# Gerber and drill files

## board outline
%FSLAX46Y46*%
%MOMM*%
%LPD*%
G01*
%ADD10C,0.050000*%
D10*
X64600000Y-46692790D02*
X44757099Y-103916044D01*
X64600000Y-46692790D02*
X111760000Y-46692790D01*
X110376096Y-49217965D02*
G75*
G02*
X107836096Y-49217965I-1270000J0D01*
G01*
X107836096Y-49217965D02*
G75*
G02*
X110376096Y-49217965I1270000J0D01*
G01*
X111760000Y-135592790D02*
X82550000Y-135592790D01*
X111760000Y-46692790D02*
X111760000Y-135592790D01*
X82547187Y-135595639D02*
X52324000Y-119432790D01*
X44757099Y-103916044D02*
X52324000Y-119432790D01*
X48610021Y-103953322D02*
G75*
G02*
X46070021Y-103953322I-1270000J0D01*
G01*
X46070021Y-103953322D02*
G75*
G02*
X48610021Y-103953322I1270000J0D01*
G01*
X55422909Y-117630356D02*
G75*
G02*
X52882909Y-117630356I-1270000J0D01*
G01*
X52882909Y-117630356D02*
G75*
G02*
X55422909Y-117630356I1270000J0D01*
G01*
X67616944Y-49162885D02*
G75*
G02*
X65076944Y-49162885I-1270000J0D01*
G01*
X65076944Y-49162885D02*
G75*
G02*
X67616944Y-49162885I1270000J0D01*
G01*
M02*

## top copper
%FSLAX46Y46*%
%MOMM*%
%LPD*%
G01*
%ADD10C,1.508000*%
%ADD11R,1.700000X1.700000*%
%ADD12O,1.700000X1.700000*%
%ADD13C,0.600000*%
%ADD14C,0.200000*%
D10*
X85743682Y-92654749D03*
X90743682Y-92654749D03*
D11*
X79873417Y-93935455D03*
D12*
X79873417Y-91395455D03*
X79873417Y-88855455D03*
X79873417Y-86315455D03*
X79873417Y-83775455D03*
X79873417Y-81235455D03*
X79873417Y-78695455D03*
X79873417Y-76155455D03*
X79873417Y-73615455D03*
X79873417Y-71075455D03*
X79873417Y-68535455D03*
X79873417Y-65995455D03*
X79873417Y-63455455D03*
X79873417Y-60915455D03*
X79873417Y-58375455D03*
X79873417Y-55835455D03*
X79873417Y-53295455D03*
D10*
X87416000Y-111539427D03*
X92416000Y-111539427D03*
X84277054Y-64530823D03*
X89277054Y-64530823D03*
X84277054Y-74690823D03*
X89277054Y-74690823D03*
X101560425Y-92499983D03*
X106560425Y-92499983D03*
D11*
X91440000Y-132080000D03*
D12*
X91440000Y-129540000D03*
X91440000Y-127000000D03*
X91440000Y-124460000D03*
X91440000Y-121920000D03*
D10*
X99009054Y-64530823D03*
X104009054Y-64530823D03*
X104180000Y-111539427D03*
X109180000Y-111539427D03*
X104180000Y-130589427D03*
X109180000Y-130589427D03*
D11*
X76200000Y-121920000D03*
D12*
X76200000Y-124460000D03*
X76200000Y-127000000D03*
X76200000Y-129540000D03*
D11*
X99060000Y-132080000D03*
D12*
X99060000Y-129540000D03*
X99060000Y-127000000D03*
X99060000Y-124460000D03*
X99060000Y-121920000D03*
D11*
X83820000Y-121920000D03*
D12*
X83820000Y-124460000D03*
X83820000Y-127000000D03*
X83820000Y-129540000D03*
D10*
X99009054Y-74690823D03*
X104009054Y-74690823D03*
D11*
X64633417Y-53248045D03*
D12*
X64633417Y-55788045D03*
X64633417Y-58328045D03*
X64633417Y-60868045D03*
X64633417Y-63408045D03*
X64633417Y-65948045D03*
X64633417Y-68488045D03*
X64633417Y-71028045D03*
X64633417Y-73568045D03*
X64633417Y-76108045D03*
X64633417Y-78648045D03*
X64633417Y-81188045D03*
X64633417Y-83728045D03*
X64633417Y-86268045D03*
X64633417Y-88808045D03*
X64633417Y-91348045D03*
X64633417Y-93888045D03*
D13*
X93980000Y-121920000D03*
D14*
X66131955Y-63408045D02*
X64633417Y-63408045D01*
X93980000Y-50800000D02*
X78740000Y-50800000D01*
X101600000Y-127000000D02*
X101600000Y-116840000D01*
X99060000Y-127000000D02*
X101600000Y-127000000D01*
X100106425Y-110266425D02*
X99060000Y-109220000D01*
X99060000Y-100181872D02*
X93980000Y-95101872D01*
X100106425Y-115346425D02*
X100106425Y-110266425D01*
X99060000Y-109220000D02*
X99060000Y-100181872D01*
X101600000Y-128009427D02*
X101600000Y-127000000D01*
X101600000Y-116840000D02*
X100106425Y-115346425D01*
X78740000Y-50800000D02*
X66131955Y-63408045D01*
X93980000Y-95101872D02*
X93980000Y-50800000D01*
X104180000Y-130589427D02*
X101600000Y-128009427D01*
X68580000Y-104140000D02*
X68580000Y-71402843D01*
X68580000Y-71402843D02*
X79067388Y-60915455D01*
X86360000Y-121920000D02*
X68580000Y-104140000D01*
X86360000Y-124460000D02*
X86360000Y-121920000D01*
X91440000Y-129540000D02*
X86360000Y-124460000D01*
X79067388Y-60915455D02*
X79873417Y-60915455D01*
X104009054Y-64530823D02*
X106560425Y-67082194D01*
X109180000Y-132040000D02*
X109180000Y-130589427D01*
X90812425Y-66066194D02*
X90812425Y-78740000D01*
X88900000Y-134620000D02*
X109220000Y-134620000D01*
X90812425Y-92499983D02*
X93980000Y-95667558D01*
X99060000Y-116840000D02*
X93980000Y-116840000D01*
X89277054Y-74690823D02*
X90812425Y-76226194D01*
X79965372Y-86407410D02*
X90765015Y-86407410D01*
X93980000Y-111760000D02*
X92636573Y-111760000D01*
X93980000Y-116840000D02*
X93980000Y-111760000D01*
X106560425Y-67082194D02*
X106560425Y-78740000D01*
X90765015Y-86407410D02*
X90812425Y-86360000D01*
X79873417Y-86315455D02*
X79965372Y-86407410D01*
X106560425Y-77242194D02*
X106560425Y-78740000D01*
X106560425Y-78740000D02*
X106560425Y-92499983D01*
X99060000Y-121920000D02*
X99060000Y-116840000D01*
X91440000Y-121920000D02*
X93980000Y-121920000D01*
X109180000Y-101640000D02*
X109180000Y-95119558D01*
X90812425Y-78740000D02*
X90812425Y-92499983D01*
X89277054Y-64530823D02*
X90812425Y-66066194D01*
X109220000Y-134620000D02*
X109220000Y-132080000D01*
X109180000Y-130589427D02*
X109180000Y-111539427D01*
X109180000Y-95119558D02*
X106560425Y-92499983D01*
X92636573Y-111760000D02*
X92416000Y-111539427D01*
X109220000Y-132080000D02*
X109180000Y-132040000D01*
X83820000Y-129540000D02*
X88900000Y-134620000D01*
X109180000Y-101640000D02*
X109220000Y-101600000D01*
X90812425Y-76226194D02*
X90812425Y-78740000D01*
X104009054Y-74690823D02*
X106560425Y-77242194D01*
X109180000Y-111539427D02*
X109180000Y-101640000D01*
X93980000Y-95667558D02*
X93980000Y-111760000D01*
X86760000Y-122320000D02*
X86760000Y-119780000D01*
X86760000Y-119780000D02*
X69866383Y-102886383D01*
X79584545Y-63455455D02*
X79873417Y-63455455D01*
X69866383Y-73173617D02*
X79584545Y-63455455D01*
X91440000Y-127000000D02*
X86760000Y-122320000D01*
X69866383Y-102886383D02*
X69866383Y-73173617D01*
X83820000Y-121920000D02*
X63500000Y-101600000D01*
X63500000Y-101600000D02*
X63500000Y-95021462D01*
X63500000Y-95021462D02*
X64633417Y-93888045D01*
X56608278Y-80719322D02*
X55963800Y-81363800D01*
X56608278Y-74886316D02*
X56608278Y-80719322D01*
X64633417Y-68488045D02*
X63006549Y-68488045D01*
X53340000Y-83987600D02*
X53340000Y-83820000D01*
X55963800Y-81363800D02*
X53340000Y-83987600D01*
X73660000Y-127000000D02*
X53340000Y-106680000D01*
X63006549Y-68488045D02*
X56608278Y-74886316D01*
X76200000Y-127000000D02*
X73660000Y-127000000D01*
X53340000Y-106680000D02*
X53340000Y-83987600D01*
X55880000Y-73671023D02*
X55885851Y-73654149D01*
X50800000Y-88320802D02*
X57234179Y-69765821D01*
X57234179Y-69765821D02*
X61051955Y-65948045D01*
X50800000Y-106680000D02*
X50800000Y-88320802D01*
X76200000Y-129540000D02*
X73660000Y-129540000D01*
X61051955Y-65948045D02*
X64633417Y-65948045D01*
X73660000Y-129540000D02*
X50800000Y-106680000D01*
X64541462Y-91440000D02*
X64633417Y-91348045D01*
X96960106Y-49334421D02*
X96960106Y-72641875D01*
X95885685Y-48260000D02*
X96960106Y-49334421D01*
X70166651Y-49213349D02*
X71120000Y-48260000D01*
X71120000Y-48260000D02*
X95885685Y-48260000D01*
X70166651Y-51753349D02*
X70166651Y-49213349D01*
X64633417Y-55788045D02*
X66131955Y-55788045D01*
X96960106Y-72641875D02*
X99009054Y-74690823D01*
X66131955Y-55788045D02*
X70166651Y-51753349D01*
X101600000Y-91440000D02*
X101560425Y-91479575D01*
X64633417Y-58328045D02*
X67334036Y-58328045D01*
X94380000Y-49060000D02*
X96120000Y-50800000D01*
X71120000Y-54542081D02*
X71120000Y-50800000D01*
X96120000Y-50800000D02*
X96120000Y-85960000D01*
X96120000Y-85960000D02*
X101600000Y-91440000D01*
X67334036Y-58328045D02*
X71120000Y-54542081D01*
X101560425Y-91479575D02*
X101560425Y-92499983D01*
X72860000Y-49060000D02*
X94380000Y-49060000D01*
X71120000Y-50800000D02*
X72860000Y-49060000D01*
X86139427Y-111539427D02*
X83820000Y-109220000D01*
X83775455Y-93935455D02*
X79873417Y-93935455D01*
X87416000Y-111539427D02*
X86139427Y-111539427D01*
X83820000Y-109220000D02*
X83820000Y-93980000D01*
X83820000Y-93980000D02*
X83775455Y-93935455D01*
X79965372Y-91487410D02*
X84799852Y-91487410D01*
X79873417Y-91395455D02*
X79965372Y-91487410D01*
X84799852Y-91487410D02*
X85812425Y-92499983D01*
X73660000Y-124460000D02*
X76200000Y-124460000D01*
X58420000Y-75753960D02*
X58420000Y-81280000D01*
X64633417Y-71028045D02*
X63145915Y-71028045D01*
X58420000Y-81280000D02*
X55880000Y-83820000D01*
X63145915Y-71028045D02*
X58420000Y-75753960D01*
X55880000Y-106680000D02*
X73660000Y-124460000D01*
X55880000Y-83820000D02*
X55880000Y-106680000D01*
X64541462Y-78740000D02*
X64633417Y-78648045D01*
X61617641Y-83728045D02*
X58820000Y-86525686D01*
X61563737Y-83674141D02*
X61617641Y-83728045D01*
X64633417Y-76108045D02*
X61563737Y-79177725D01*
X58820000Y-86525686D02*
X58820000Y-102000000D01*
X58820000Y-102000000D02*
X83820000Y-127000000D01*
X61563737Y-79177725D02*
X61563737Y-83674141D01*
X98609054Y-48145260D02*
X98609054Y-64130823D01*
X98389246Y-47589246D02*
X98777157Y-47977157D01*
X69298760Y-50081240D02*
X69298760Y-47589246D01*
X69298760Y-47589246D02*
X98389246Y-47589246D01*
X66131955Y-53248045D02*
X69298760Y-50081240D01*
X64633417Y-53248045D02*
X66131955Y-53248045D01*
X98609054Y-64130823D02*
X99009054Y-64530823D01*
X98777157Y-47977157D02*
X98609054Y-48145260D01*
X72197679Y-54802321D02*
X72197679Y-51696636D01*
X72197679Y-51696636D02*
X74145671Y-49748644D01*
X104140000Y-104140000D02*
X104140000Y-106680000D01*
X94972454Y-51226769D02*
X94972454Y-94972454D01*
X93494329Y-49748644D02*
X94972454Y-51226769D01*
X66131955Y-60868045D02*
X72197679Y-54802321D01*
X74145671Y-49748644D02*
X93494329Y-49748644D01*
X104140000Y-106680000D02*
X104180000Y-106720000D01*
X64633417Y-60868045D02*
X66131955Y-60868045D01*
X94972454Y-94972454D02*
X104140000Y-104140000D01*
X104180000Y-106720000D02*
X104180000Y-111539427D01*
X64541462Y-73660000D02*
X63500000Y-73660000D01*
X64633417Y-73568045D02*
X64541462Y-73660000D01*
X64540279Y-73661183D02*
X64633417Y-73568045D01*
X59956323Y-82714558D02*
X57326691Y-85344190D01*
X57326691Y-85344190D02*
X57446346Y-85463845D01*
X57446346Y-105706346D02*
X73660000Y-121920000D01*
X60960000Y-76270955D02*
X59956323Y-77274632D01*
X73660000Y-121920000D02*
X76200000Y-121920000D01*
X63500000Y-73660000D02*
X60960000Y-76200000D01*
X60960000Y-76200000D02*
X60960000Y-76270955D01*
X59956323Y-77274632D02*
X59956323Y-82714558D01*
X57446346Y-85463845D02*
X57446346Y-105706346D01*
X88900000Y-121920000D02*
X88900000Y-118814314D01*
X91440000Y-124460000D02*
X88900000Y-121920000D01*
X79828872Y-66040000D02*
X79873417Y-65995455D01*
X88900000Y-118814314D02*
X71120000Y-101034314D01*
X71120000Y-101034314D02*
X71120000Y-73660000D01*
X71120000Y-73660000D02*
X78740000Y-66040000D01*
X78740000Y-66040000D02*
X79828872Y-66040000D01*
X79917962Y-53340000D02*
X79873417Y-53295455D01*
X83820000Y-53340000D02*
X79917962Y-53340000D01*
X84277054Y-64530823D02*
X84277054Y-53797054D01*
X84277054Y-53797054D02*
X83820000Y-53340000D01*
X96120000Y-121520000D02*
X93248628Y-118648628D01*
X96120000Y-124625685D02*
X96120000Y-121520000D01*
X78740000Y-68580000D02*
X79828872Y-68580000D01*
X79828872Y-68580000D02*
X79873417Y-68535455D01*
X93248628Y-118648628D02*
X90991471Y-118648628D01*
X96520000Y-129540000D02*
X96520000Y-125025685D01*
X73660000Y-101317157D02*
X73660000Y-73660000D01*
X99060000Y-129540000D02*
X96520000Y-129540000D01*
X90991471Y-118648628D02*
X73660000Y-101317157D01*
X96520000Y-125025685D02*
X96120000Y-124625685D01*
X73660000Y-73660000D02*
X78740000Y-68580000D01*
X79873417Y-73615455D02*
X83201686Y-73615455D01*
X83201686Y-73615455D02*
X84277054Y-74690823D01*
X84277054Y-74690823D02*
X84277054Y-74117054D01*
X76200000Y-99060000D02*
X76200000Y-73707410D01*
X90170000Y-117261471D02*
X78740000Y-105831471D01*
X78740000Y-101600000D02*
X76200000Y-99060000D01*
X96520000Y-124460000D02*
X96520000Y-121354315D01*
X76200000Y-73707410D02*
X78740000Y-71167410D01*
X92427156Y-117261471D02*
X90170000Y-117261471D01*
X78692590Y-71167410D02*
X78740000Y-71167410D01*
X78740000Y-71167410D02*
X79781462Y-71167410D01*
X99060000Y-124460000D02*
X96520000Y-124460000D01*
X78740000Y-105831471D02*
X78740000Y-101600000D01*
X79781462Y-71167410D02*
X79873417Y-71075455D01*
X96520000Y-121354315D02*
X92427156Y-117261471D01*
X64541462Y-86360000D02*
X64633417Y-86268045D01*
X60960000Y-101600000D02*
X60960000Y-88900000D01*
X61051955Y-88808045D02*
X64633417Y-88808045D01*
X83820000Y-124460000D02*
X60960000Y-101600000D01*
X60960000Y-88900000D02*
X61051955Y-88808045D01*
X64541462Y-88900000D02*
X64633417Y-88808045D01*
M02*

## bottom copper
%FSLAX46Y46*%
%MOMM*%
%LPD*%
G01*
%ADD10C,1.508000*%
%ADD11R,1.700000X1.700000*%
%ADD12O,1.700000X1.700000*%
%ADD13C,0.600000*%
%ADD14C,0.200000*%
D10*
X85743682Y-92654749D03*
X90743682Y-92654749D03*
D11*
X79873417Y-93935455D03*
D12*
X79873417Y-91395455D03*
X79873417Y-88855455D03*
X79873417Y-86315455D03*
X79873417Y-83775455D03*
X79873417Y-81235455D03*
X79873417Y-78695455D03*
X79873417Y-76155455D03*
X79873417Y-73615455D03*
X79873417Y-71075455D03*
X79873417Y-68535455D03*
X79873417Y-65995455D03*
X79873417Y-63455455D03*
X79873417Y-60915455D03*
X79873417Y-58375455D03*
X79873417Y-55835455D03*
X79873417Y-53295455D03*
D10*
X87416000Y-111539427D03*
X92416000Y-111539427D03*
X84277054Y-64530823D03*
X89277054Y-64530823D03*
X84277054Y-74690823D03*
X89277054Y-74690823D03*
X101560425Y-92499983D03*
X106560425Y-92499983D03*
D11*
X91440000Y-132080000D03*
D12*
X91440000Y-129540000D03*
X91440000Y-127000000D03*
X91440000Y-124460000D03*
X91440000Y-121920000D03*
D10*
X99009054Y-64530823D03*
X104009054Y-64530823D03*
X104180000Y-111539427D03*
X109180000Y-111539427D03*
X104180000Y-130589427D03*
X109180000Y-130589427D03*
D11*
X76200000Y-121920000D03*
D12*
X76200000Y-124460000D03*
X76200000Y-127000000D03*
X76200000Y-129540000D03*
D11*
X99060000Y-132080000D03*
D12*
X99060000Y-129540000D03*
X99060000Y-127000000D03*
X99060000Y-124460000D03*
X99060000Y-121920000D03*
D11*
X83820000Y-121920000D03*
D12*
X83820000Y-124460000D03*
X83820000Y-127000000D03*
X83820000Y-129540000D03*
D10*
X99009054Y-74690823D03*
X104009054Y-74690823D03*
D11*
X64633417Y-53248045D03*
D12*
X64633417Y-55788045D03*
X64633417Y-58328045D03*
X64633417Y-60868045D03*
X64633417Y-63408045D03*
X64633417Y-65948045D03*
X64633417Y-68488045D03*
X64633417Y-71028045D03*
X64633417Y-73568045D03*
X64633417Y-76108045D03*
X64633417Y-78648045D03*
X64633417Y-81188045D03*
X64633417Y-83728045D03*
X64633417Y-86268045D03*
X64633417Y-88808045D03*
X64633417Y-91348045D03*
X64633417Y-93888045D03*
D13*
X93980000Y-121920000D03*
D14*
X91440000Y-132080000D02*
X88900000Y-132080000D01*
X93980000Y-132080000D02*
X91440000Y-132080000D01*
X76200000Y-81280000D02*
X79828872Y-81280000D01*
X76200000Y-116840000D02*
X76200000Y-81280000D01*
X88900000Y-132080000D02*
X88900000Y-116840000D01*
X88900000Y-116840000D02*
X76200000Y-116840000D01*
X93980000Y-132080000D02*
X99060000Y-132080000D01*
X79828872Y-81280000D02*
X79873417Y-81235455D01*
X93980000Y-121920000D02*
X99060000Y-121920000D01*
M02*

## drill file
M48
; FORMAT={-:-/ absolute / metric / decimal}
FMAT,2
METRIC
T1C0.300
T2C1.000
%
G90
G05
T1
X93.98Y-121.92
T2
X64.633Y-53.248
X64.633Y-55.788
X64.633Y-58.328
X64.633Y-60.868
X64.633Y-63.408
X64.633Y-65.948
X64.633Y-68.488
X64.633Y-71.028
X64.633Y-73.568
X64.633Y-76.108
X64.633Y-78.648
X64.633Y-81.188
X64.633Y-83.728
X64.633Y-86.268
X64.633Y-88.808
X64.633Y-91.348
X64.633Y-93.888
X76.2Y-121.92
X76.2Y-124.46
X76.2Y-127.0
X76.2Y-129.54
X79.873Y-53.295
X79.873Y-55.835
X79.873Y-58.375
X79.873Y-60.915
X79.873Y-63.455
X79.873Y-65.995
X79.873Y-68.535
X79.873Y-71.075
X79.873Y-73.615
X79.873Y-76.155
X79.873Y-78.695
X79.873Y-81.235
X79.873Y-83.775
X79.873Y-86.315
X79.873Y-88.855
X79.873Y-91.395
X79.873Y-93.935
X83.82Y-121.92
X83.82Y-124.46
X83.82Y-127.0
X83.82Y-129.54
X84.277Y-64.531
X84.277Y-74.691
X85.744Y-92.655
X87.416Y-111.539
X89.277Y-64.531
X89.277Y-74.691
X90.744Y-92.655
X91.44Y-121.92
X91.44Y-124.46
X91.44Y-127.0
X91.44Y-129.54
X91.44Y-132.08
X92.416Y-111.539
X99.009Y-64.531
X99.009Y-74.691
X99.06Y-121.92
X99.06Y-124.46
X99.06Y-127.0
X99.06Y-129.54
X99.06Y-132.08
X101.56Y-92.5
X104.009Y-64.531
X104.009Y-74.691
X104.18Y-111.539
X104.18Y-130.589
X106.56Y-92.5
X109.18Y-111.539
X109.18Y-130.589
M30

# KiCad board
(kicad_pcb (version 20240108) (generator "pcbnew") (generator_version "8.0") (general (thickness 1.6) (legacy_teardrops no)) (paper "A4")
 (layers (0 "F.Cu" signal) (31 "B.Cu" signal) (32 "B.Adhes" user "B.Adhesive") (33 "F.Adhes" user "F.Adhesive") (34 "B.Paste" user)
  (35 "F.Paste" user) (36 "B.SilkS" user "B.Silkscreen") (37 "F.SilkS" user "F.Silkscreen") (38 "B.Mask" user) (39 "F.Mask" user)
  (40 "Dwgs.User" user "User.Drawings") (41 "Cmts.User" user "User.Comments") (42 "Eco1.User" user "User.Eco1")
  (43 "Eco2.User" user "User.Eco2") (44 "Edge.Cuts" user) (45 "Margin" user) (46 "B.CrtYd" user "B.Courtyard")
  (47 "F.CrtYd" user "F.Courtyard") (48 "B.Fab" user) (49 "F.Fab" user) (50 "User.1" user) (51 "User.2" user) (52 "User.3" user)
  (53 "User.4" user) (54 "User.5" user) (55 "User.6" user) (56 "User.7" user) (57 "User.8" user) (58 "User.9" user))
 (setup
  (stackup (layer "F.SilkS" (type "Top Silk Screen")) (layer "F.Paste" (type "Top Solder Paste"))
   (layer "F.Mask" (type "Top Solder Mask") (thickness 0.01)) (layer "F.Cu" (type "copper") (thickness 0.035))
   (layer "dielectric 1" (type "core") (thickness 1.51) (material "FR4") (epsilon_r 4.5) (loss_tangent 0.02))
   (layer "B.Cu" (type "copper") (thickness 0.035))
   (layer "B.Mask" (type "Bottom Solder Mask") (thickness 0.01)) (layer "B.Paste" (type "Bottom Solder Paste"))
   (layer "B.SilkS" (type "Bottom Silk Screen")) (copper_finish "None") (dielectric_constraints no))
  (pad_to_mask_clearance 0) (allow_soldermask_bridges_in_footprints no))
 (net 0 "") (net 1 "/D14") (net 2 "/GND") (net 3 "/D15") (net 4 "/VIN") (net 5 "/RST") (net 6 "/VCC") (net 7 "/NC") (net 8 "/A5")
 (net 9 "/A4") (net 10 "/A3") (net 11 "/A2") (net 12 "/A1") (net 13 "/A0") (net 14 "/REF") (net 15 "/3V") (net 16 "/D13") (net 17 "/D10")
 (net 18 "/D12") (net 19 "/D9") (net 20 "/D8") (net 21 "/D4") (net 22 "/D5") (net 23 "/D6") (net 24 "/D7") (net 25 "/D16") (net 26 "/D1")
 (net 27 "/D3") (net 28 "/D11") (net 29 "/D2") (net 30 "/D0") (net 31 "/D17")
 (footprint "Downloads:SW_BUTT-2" (layer "F.Cu") (at 88.243682 92.654749)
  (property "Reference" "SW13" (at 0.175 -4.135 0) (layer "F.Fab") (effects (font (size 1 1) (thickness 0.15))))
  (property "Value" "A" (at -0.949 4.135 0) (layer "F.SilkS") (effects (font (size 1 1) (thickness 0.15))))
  (pad "1" thru_hole circle (at -2.5 0) (size 1.508 1.508) (drill 1) (layers "*.Cu" "*.Mask") (remove_unused_layers no) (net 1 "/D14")
   (solder_mask_margin 0.102))
  (pad "2" thru_hole circle (at 2.5 0) (size 1.508 1.508) (drill 1) (layers "*.Cu" "*.Mask") (remove_unused_layers no) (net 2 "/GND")
   (solder_mask_margin 0.102)))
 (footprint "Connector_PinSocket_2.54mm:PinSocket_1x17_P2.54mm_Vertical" (layer "F.Cu") (at 79.873417 93.935455 180)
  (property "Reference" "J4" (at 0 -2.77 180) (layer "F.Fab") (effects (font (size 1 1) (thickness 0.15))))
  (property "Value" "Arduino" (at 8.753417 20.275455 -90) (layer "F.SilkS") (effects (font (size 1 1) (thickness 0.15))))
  (pad "1" thru_hole rect (at 0 0 180) (size 1.7 1.7) (drill 1) (layers "*.Cu" "*.Mask") (remove_unused_layers no) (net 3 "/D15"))
  (pad "2" thru_hole oval (at 0 2.54 180) (size 1.7 1.7) (drill 1) (layers "*.Cu" "*.Mask") (remove_unused_layers no) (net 1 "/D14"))
  (pad "3" thru_hole oval (at 0 5.08 180) (size 1.7 1.7) (drill 1) (layers "*.Cu" "*.Mask") (remove_unused_layers no) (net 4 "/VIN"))
  (pad "4" thru_hole oval (at 0 7.62 180) (size 1.7 1.7) (drill 1) (layers "*.Cu" "*.Mask") (remove_unused_layers no) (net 2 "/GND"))
  (pad "5" thru_hole oval (at 0 10.16 180) (size 1.7 1.7) (drill 1) (layers "*.Cu" "*.Mask") (remove_unused_layers no) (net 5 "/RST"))
  (pad "6" thru_hole oval (at 0 12.7 180) (size 1.7 1.7) (drill 1) (layers "*.Cu" "*.Mask") (remove_unused_layers no) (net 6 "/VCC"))
  (pad "7" thru_hole oval (at 0 15.24 180) (size 1.7 1.7) (drill 1) (layers "*.Cu" "*.Mask") (remove_unused_layers no) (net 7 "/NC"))
  (pad "8" thru_hole oval (at 0 17.78 180) (size 1.7 1.7) (drill 1) (layers "*.Cu" "*.Mask") (remove_unused_layers no) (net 7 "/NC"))
  (pad "9" thru_hole oval (at 0 20.32 180) (size 1.7 1.7) (drill 1) (layers "*.Cu" "*.Mask") (remove_unused_layers no) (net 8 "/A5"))
  (pad "10" thru_hole oval (at 0 22.86 180) (size 1.7 1.7) (drill 1) (layers "*.Cu" "*.Mask") (remove_unused_layers no) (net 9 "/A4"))
  (pad "11" thru_hole oval (at 0 25.4 180) (size 1.7 1.7) (drill 1) (layers "*.Cu" "*.Mask") (remove_unused_layers no) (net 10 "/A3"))
  (pad "12" thru_hole oval (at 0 27.94 180) (size 1.7 1.7) (drill 1) (layers "*.Cu" "*.Mask") (remove_unused_layers no) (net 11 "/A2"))
  (pad "13" thru_hole oval (at 0 30.48 180) (size 1.7 1.7) (drill 1) (layers "*.Cu" "*.Mask") (remove_unused_layers no) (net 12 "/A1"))
  (pad "14" thru_hole oval (at 0 33.02 180) (size 1.7 1.7) (drill 1) (layers "*.Cu" "*.Mask") (remove_unused_layers no) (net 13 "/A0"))
  (pad "15" thru_hole oval (at 0 35.56 180) (size 1.7 1.7) (drill 1) (layers "*.Cu" "*.Mask") (remove_unused_layers no) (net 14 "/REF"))
  (pad "16" thru_hole oval (at 0 38.1 180) (size 1.7 1.7) (drill 1) (layers "*.Cu" "*.Mask") (remove_unused_layers no) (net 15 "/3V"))
  (pad "17" thru_hole oval (at 0 40.64 180) (size 1.7 1.7) (drill 1) (layers "*.Cu" "*.Mask") (remove_unused_layers no) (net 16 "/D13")))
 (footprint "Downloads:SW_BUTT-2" (layer "F.Cu") (at 89.916 111.539427)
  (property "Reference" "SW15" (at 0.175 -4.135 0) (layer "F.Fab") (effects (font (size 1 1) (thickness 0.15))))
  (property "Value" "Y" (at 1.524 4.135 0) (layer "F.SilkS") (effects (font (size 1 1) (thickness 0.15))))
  (pad "1" thru_hole circle (at -2.5 0) (size 1.508 1.508) (drill 1) (layers "*.Cu" "*.Mask") (remove_unused_layers no) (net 3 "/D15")
   (solder_mask_margin 0.102))
  (pad "2" thru_hole circle (at 2.5 0) (size 1.508 1.508) (drill 1) (layers "*.Cu" "*.Mask") (remove_unused_layers no) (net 2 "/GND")
   (solder_mask_margin 0.102)))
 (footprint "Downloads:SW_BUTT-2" (layer "F.Cu") (at 86.777054 64.530823)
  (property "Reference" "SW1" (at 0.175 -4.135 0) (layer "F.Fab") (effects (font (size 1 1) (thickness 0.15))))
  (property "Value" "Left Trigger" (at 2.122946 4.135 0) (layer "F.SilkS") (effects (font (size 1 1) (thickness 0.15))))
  (pad "1" thru_hole circle (at -2.5 0) (size 1.508 1.508) (drill 1) (layers "*.Cu" "*.Mask") (remove_unused_layers no) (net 16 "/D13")
   (solder_mask_margin 0.102))
  (pad "2" thru_hole circle (at 2.5 0) (size 1.508 1.508) (drill 1) (layers "*.Cu" "*.Mask") (remove_unused_layers no) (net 2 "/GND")
   (solder_mask_margin 0.102)))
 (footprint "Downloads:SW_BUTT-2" (layer "F.Cu") (at 86.777054 74.690823)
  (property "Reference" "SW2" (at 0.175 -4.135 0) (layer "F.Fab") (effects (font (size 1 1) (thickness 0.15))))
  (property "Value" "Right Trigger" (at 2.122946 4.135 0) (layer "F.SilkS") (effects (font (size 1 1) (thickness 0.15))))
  (pad "1" thru_hole circle (at -2.5 0) (size 1.508 1.508) (drill 1) (layers "*.Cu" "*.Mask") (remove_unused_layers no) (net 8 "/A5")
   (solder_mask_margin 0.102))
  (pad "2" thru_hole circle (at 2.5 0) (size 1.508 1.508) (drill 1) (layers "*.Cu" "*.Mask") (remove_unused_layers no) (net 2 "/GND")
   (solder_mask_margin 0.102)))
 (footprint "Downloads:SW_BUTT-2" (layer "F.Cu") (at 104.060425 92.499983)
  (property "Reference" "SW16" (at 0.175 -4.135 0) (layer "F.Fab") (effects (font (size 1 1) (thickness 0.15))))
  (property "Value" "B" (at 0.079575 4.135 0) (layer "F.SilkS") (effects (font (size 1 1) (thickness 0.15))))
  (pad "1" thru_hole circle (at -2.5 0) (size 1.508 1.508) (drill 1) (layers "*.Cu" "*.Mask") (remove_unused_layers no) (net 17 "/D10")
   (solder_mask_margin 0.102))
  (pad "2" thru_hole circle (at 2.5 0) (size 1.508 1.508) (drill 1) (layers "*.Cu" "*.Mask") (remove_unused_layers no) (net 2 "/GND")
   (solder_mask_margin 0.102)))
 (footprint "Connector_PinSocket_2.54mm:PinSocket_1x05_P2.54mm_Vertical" (layer "F.Cu") (at 91.44 132.08 180)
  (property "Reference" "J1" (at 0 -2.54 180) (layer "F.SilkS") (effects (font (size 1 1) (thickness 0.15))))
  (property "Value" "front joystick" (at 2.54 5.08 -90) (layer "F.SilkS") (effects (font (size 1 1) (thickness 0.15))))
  (pad "1" thru_hole rect (at 0 0 180) (size 1.7 1.7) (drill 1) (layers "*.Cu" "*.Mask") (remove_unused_layers no) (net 6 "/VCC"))
  (pad "2" thru_hole oval (at 0 2.54 180) (size 1.7 1.7) (drill 1) (layers "*.Cu" "*.Mask") (remove_unused_layers no) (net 13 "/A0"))
  (pad "3" thru_hole oval (at 0 5.08 180) (size 1.7 1.7) (drill 1) (layers "*.Cu" "*.Mask") (remove_unused_layers no) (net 12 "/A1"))
  (pad "4" thru_hole oval (at 0 7.62 180) (size 1.7 1.7) (drill 1) (layers "*.Cu" "*.Mask") (remove_unused_layers no) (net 11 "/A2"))
  (pad "5" thru_hole oval (at 0 10.16 180) (size 1.7 1.7) (drill 1) (layers "*.Cu" "*.Mask") (remove_unused_layers no) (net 2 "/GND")))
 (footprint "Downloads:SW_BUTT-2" (layer "F.Cu") (at 101.509054 64.530823)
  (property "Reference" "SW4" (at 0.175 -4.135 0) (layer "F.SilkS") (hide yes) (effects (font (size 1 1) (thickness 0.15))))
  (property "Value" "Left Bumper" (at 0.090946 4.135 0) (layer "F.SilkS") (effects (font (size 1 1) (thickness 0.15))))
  (pad "1" thru_hole circle (at -2.5 0) (size 1.508 1.508) (drill 1) (layers "*.Cu" "*.Mask") (remove_unused_layers no) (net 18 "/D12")
   (solder_mask_margin 0.102))
  (pad "2" thru_hole circle (at 2.5 0) (size 1.508 1.508) (drill 1) (layers "*.Cu" "*.Mask") (remove_unused_layers no) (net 2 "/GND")
   (solder_mask_margin 0.102)))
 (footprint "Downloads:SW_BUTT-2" (layer "F.Cu") (at 106.68 111.539427)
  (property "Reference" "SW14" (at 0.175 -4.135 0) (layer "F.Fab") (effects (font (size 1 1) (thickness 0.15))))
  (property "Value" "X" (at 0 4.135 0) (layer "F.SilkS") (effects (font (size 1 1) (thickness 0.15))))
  (pad "1" thru_hole circle (at -2.5 0) (size 1.508 1.508) (drill 1) (layers "*.Cu" "*.Mask") (remove_unused_layers no) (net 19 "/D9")
   (solder_mask_margin 0.102))
  (pad "2" thru_hole circle (at 2.5 0) (size 1.508 1.508) (drill 1) (layers "*.Cu" "*.Mask") (remove_unused_layers no) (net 2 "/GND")
   (solder_mask_margin 0.102)))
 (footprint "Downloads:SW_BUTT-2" (layer "F.Cu") (at 106.68 130.589427)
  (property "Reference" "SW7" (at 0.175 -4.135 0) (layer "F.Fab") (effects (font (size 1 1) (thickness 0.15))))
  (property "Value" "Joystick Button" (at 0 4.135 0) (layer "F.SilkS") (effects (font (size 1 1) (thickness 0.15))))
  (pad "1" thru_hole circle (at -2.5 0) (size 1.508 1.508) (drill 1) (layers "*.Cu" "*.Mask") (remove_unused_layers no) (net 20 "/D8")
   (solder_mask_margin 0.102))
  (pad "2" thru_hole circle (at 2.5 0) (size 1.508 1.508) (drill 1) (layers "*.Cu" "*.Mask") (remove_unused_layers no) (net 2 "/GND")
   (solder_mask_margin 0.102)))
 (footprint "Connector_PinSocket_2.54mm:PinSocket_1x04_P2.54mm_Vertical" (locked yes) (layer "F.Cu") (at 76.2 121.92)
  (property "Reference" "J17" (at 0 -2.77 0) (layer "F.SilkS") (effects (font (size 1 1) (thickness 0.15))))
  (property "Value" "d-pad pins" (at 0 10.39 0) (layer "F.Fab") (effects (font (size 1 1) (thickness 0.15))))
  (pad "1" thru_hole rect (at 0 0) (size 1.7 1.7) (drill 1) (layers "*.Cu" "*.Mask") (remove_unused_layers no) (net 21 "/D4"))
  (pad "2" thru_hole oval (at 0 2.54) (size 1.7 1.7) (drill 1) (layers "*.Cu" "*.Mask") (remove_unused_layers no) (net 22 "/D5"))
  (pad "3" thru_hole oval (at 0 5.08) (size 1.7 1.7) (drill 1) (layers "*.Cu" "*.Mask") (remove_unused_layers no) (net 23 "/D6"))
  (pad "4" thru_hole oval (at 0 7.62) (size 1.7 1.7) (drill 1) (layers "*.Cu" "*.Mask") (remove_unused_layers no) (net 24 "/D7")))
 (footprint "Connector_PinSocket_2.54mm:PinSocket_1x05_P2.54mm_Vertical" (layer "F.Cu") (at 99.06 132.08 180)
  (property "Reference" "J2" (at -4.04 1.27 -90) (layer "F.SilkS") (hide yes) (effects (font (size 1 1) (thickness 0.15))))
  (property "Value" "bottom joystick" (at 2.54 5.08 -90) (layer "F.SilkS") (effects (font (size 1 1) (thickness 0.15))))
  (pad "1" thru_hole rect (at 0 0 180) (size 1.7 1.7) (drill 1) (layers "*.Cu" "*.Mask") (remove_unused_layers no) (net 6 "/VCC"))
  (pad "2" thru_hole oval (at 0 2.54 180) (size 1.7 1.7) (drill 1) (layers "*.Cu" "*.Mask") (remove_unused_layers no) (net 10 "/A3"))
  (pad "3" thru_hole oval (at 0 5.08 180) (size 1.7 1.7) (drill 1) (layers "*.Cu" "*.Mask") (remove_unused_layers no) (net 20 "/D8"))
  (pad "4" thru_hole oval (at 0 7.62 180) (size 1.7 1.7) (drill 1) (layers "*.Cu" "*.Mask") (remove_unused_layers no) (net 9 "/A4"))
  (pad "5" thru_hole oval (at 0 10.16 180) (size 1.7 1.7) (drill 1) (layers "*.Cu" "*.Mask") (remove_unused_layers no) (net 2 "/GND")))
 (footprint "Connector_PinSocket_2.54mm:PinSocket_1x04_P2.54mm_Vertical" (layer "F.Cu") (at 83.82 121.92)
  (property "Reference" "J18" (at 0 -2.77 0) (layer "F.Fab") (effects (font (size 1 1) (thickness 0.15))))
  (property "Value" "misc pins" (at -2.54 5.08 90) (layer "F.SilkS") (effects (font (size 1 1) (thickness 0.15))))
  (pad "1" thru_hole rect (at 0 0) (size 1.7 1.7) (drill 1) (layers "*.Cu" "*.Mask") (remove_unused_layers no) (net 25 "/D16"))
  (pad "2" thru_hole oval (at 0 2.54) (size 1.7 1.7) (drill 1) (layers "*.Cu" "*.Mask") (remove_unused_layers no) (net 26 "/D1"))
  (pad "3" thru_hole oval (at 0 5.08) (size 1.7 1.7) (drill 1) (layers "*.Cu" "*.Mask") (remove_unused_layers no) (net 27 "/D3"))
  (pad "4" thru_hole oval (at 0 7.62) (size 1.7 1.7) (drill 1) (layers "*.Cu" "*.Mask") (remove_unused_layers no) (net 2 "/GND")))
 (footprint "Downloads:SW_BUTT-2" (layer "F.Cu") (at 101.509054 74.690823)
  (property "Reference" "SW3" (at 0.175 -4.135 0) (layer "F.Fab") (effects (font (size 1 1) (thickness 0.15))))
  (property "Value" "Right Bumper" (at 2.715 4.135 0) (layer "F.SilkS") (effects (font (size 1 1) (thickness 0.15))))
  (pad "1" thru_hole circle (at -2.5 0) (size 1.508 1.508) (drill 1) (layers "*.Cu" "*.Mask") (remove_unused_layers no) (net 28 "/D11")
   (solder_mask_margin 0.102))
  (pad "2" thru_hole circle (at 2.5 0) (size 1.508 1.508) (drill 1) (layers "*.Cu" "*.Mask") (remove_unused_layers no) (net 2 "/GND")
   (solder_mask_margin 0.102)))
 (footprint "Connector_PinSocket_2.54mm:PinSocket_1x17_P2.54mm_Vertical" (layer "F.Cu") (at 64.633417 53.248045)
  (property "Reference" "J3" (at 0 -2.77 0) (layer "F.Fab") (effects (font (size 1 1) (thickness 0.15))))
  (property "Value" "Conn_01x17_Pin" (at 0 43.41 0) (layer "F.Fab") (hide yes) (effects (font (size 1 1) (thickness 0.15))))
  (pad "1" thru_hole rect (at 0 0) (size 1.7 1.7) (drill 1) (layers "*.Cu" "*.Mask") (remove_unused_layers no) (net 18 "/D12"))
  (pad "2" thru_hole oval (at 0 2.54) (size 1.7 1.7) (drill 1) (layers "*.Cu" "*.Mask") (remove_unused_layers no) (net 28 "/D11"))
  (pad "3" thru_hole oval (at 0 5.08) (size 1.7 1.7) (drill 1) (layers "*.Cu" "*.Mask") (remove_unused_layers no) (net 17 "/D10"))
  (pad "4" thru_hole oval (at 0 7.62) (size 1.7 1.7) (drill 1) (layers "*.Cu" "*.Mask") (remove_unused_layers no) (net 19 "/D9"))
  (pad "5" thru_hole oval (at 0 10.16) (size 1.7 1.7) (drill 1) (layers "*.Cu" "*.Mask") (remove_unused_layers no) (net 20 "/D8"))
  (pad "6" thru_hole oval (at 0 12.7) (size 1.7 1.7) (drill 1) (layers "*.Cu" "*.Mask") (remove_unused_layers no) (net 24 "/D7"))
  (pad "7" thru_hole oval (at 0 15.24) (size 1.7 1.7) (drill 1) (layers "*.Cu" "*.Mask") (remove_unused_layers no) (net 23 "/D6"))
  (pad "8" thru_hole oval (at 0 17.78) (size 1.7 1.7) (drill 1) (layers "*.Cu" "*.Mask") (remove_unused_layers no) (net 22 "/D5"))
  (pad "9" thru_hole oval (at 0 20.32) (size 1.7 1.7) (drill 1) (layers "*.Cu" "*.Mask") (remove_unused_layers no) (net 21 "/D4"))
  (pad "10" thru_hole oval (at 0 22.86) (size 1.7 1.7) (drill 1) (layers "*.Cu" "*.Mask") (remove_unused_layers no) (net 27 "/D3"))
  (pad "11" thru_hole oval (at 0 25.4) (size 1.7 1.7) (drill 1) (layers "*.Cu" "*.Mask") (remove_unused_layers no) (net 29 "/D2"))
  (pad "12" thru_hole oval (at 0 27.94) (size 1.7 1.7) (drill 1) (layers "*.Cu" "*.Mask") (remove_unused_layers no) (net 2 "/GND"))
  (pad "13" thru_hole oval (at 0 30.48) (size 1.7 1.7) (drill 1) (layers "*.Cu" "*.Mask") (remove_unused_layers no) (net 5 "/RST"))
  (pad "14" thru_hole oval (at 0 33.02) (size 1.7 1.7) (drill 1) (layers "*.Cu" "*.Mask") (remove_unused_layers no) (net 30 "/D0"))
  (pad "15" thru_hole oval (at 0 35.56) (size 1.7 1.7) (drill 1) (layers "*.Cu" "*.Mask") (remove_unused_layers no) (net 26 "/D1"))
  (pad "16" thru_hole oval (at 0 38.1) (size 1.7 1.7) (drill 1) (layers "*.Cu" "*.Mask") (remove_unused_layers no) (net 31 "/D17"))
  (pad "17" thru_hole oval (at 0 40.64) (size 1.7 1.7) (drill 1) (layers "*.Cu" "*.Mask") (remove_unused_layers no) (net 25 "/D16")))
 (gr_line (start 64.6 46.69279) (end 44.757099 103.916044) (stroke (width 0.05) (type default)) (layer "Edge.Cuts"))
 (gr_line (start 64.6 46.69279) (end 111.76 46.69279) (stroke (width 0.05) (type default)) (layer "Edge.Cuts"))
 (gr_circle (center 109.106096 49.217965) (end 110.376096 49.217965) (stroke (width 0.05) (type default)) (fill none) (layer "Edge.Cuts"))
 (gr_line (start 111.76 135.59279) (end 82.55 135.59279) (stroke (width 0.05) (type default)) (layer "Edge.Cuts"))
 (gr_line (start 111.76 46.69279) (end 111.76 135.59279) (stroke (width 0.05) (type default)) (layer "Edge.Cuts"))
 (gr_line (start 82.547187 135.595639) (end 52.324 119.43279) (stroke (width 0.05) (type default)) (layer "Edge.Cuts"))
 (gr_line (start 44.757099 103.916044) (end 52.324 119.43279) (stroke (width 0.05) (type default)) (layer "Edge.Cuts"))
 (gr_circle (center 47.340021 103.953322) (end 46.070021 103.953322) (stroke (width 0.05) (type default)) (fill none) (layer "Edge.Cuts"))
 (gr_circle (center 54.152909 117.630356) (end 52.882909 117.630356) (stroke (width 0.05) (type default)) (fill none) (layer "Edge.Cuts"))
 (gr_circle (center 66.346944 49.162885) (end 66.346944 47.892885) (stroke (width 0.05) (type default)) (fill none) (layer "Edge.Cuts"))
 (segment (start 66.131955 63.408045) (end 64.633417 63.408045) (width 0.2) (layer "F.Cu") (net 20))
 (segment (start 93.98 50.8) (end 78.74 50.8) (width 0.2) (layer "F.Cu") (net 20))
 (segment (start 101.6 127) (end 101.6 116.84) (width 0.2) (layer "F.Cu") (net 20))
 (segment (start 99.06 127) (end 101.6 127) (width 0.2) (layer "F.Cu") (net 20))
 (segment (start 100.106425 110.266425) (end 99.06 109.22) (width 0.2) (layer "F.Cu") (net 20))
 (segment (start 99.06 100.181872) (end 93.98 95.101872) (width 0.2) (layer "F.Cu") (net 20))
 (segment (start 100.106425 115.346425) (end 100.106425 110.266425) (width 0.2) (layer "F.Cu") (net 20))
 (segment (start 99.06 109.22) (end 99.06 100.181872) (width 0.2) (layer "F.Cu") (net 20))
 (segment (start 101.6 128.009427) (end 101.6 127) (width 0.2) (layer "F.Cu") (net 20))
 (segment (start 101.6 116.84) (end 100.106425 115.346425) (width 0.2) (layer "F.Cu") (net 20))
 (segment (start 78.74 50.8) (end 66.131955 63.408045) (width 0.2) (layer "F.Cu") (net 20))
 (segment (start 93.98 95.101872) (end 93.98 50.8) (width 0.2) (layer "F.Cu") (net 20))
 (segment (start 104.18 130.589427) (end 101.6 128.009427) (width 0.2) (layer "F.Cu") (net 20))
 (segment (start 91.44 132.08) (end 88.9 132.08) (width 0.2) (layer "B.Cu") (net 6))
 (segment (start 93.98 132.08) (end 91.44 132.08) (width 0.2) (layer "B.Cu") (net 6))
 (segment (start 76.2 81.28) (end 79.828872 81.28) (width 0.2) (layer "B.Cu") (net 6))
 (segment (start 76.2 116.84) (end 76.2 81.28) (width 0.2) (layer "B.Cu") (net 6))
 (segment (start 88.9 132.08) (end 88.9 116.84) (width 0.2) (layer "B.Cu") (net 6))
 (segment (start 88.9 116.84) (end 76.2 116.84) (width 0.2) (layer "B.Cu") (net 6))
 (segment (start 93.98 132.08) (end 99.06 132.08) (width 0.2) (layer "B.Cu") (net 6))
 (segment (start 79.828872 81.28) (end 79.873417 81.235455) (width 0.2) (layer "B.Cu") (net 6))
 (segment (start 68.58 104.14) (end 68.58 71.402843) (width 0.2) (layer "F.Cu") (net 13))
 (segment (start 68.58 71.402843) (end 79.067388 60.915455) (width 0.2) (layer "F.Cu") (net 13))
 (segment (start 86.36 121.92) (end 68.58 104.14) (width 0.2) (layer "F.Cu") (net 13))
 (segment (start 86.36 124.46) (end 86.36 121.92) (width 0.2) (layer "F.Cu") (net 13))
 (segment (start 91.44 129.54) (end 86.36 124.46) (width 0.2) (layer "F.Cu") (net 13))
 (segment (start 79.067388 60.915455) (end 79.873417 60.915455) (width 0.2) (layer "F.Cu") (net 13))
 (segment (start 104.009054 64.530823) (end 106.560425 67.082194) (width 0.2) (layer "F.Cu") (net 2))
 (segment (start 109.18 132.04) (end 109.18 130.589427) (width 0.2) (layer "F.Cu") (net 2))
 (segment (start 90.812425 66.066194) (end 90.812425 78.74) (width 0.2) (layer "F.Cu") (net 2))
 (segment (start 88.9 134.62) (end 109.22 134.62) (width 0.2) (layer "F.Cu") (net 2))
 (segment (start 90.812425 92.499983) (end 93.98 95.667558) (width 0.2) (layer "F.Cu") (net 2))
 (segment (start 99.06 116.84) (end 93.98 116.84) (width 0.2) (layer "F.Cu") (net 2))
 (segment (start 89.277054 74.690823) (end 90.812425 76.226194) (width 0.2) (layer "F.Cu") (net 2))
 (segment (start 79.965372 86.40741) (end 90.765015 86.40741) (width 0.2) (layer "F.Cu") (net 2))
 (segment (start 93.98 111.76) (end 92.636573 111.76) (width 0.2) (layer "F.Cu") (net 2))
 (segment (start 93.98 116.84) (end 93.98 111.76) (width 0.2) (layer "F.Cu") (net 2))
 (segment (start 106.560425 67.082194) (end 106.560425 78.74) (width 0.2) (layer "F.Cu") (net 2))
 (segment (start 90.765015 86.40741) (end 90.812425 86.36) (width 0.2) (layer "F.Cu") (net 2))
 (segment (start 79.873417 86.315455) (end 79.965372 86.40741) (width 0.2) (layer "F.Cu") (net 2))
 (segment (start 106.560425 77.242194) (end 106.560425 78.74) (width 0.2) (layer "F.Cu") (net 2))
 (segment (start 106.560425 78.74) (end 106.560425 92.499983) (width 0.2) (layer "F.Cu") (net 2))
 (segment (start 99.06 121.92) (end 99.06 116.84) (width 0.2) (layer "F.Cu") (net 2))
 (segment (start 91.44 121.92) (end 93.98 121.92) (width 0.2) (layer "F.Cu") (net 2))
 (segment (start 109.18 101.64) (end 109.18 95.119558) (width 0.2) (layer "F.Cu") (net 2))
 (segment (start 90.812425 78.74) (end 90.812425 92.499983) (width 0.2) (layer "F.Cu") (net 2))
 (segment (start 89.277054 64.530823) (end 90.812425 66.066194) (width 0.2) (layer "F.Cu") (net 2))
 (segment (start 109.22 134.62) (end 109.22 132.08) (width 0.2) (layer "F.Cu") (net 2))
 (segment (start 109.18 130.589427) (end 109.18 111.539427) (width 0.2) (layer "F.Cu") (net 2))
 (segment (start 109.18 95.119558) (end 106.560425 92.499983) (width 0.2) (layer "F.Cu") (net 2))
 (segment (start 92.636573 111.76) (end 92.416 111.539427) (width 0.2) (layer "F.Cu") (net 2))
 (segment (start 109.22 132.08) (end 109.18 132.04) (width 0.2) (layer "F.Cu") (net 2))
 (segment (start 83.82 129.54) (end 88.9 134.62) (width 0.2) (layer "F.Cu") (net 2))
 (segment (start 109.18 101.64) (end 109.22 101.6) (width 0.2) (layer "F.Cu") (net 2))
 (segment (start 90.812425 76.226194) (end 90.812425 78.74) (width 0.2) (layer "F.Cu") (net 2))
 (segment (start 104.009054 74.690823) (end 106.560425 77.242194) (width 0.2) (layer "F.Cu") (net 2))
 (segment (start 109.18 111.539427) (end 109.18 101.64) (width 0.2) (layer "F.Cu") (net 2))
 (segment (start 93.98 95.667558) (end 93.98 111.76) (width 0.2) (layer "F.Cu") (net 2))
 (via (at 93.98 121.92) (size 0.6) (drill 0.3) (layers "F.Cu" "B.Cu") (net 2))
 (segment (start 93.98 121.92) (end 99.06 121.92) (width 0.2) (layer "B.Cu") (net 2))
 (segment (start 86.76 122.32) (end 86.76 119.78) (width 0.2) (layer "F.Cu") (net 12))
 (segment (start 86.76 119.78) (end 69.866383 102.886383) (width 0.2) (layer "F.Cu") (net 12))
 (segment (start 79.584545 63.455455) (end 79.873417 63.455455) (width 0.2) (layer "F.Cu") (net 12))
 (segment (start 69.866383 73.173617) (end 79.584545 63.455455) (width 0.2) (layer "F.Cu") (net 12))
 (segment (start 91.44 127) (end 86.76 122.32) (width 0.2) (layer "F.Cu") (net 12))
 (segment (start 69.866383 102.886383) (end 69.866383 73.173617) (width 0.2) (layer "F.Cu") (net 12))
 (segment (start 83.82 121.92) (end 63.5 101.6) (width 0.2) (layer "F.Cu") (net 25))
 (segment (start 63.5 101.6) (end 63.5 95.021462) (width 0.2) (layer "F.Cu") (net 25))
 (segment (start 63.5 95.021462) (end 64.633417 93.888045) (width 0.2) (layer "F.Cu") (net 25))
 (segment (start 56.608278 80.719322) (end 55.9638 81.3638) (width 0.2) (layer "F.Cu") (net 23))
 (segment (start 56.608278 74.886316) (end 56.608278 80.719322) (width 0.2) (layer "F.Cu") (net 23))
 (segment (start 64.633417 68.488045) (end 63.006549 68.488045) (width 0.2) (layer "F.Cu") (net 23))
 (segment (start 53.34 83.9876) (end 53.34 83.82) (width 0.2) (layer "F.Cu") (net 23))
 (segment (start 55.9638 81.3638) (end 53.34 83.9876) (width 0.2) (layer "F.Cu") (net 23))
 (segment (start 73.66 127) (end 53.34 106.68) (width 0.2) (layer "F.Cu") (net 23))
 (segment (start 63.006549 68.488045) (end 56.608278 74.886316) (width 0.2) (layer "F.Cu") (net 23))
 (segment (start 76.2 127) (end 73.66 127) (width 0.2) (layer "F.Cu") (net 23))
 (segment (start 53.34 106.68) (end 53.34 83.9876) (width 0.2) (layer "F.Cu") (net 23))
 (segment (start 55.88 73.671023) (end 55.885851 73.654149) (width 0.2) (layer "F.Cu") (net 24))
 (segment (start 50.8 88.320802) (end 57.234179 69.765821) (width 0.2) (layer "F.Cu") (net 24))
 (segment (start 57.234179 69.765821) (end 61.051955 65.948045) (width 0.2) (layer "F.Cu") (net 24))
 (segment (start 50.8 106.68) (end 50.8 88.320802) (width 0.2) (layer "F.Cu") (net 24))
 (segment (start 76.2 129.54) (end 73.66 129.54) (width 0.2) (layer "F.Cu") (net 24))
 (segment (start 61.051955 65.948045) (end 64.633417 65.948045) (width 0.2) (layer "F.Cu") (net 24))
 (segment (start 73.66 129.54) (end 50.8 106.68) (width 0.2) (layer "F.Cu") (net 24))
 (segment (start 64.541462 91.44) (end 64.633417 91.348045) (width 0.2) (layer "F.Cu") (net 31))
 (segment (start 96.960106 49.334421) (end 96.960106 72.641875) (width 0.2) (layer "F.Cu") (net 28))
 (segment (start 95.885685 48.26) (end 96.960106 49.334421) (width 0.2) (layer "F.Cu") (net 28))
 (segment (start 70.166651 49.213349) (end 71.12 48.26) (width 0.2) (layer "F.Cu") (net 28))
 (segment (start 71.12 48.26) (end 95.885685 48.26) (width 0.2) (layer "F.Cu") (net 28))
 (segment (start 70.166651 51.753349) (end 70.166651 49.213349) (width 0.2) (layer "F.Cu") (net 28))
 (segment (start 64.633417 55.788045) (end 66.131955 55.788045) (width 0.2) (layer "F.Cu") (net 28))
 (segment (start 96.960106 72.641875) (end 99.009054 74.690823) (width 0.2) (layer "F.Cu") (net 28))
 (segment (start 66.131955 55.788045) (end 70.166651 51.753349) (width 0.2) (layer "F.Cu") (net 28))
 (segment (start 101.6 91.44) (end 101.560425 91.479575) (width 0.2) (layer "F.Cu") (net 17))
 (segment (start 64.633417 58.328045) (end 67.334036 58.328045) (width 0.2) (layer "F.Cu") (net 17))
 (segment (start 94.38 49.06) (end 96.12 50.8) (width 0.2) (layer "F.Cu") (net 17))
 (segment (start 71.12 54.542081) (end 71.12 50.8) (width 0.2) (layer "F.Cu") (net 17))
 (segment (start 96.12 50.8) (end 96.12 85.96) (width 0.2) (layer "F.Cu") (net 17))
 (segment (start 96.12 85.96) (end 101.6 91.44) (width 0.2) (layer "F.Cu") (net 17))
 (segment (start 67.334036 58.328045) (end 71.12 54.542081) (width 0.2) (layer "F.Cu") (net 17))
 (segment (start 101.560425 91.479575) (end 101.560425 92.499983) (width 0.2) (layer "F.Cu") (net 17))
 (segment (start 72.86 49.06) (end 94.38 49.06) (width 0.2) (layer "F.Cu") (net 17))
 (segment (start 71.12 50.8) (end 72.86 49.06) (width 0.2) (layer "F.Cu") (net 17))
 (segment (start 86.139427 111.539427) (end 83.82 109.22) (width 0.2) (layer "F.Cu") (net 3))
 (segment (start 83.775455 93.935455) (end 79.873417 93.935455) (width 0.2) (layer "F.Cu") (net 3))
 (segment (start 87.416 111.539427) (end 86.139427 111.539427) (width 0.2) (layer "F.Cu") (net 3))
 (segment (start 83.82 109.22) (end 83.82 93.98) (width 0.2) (layer "F.Cu") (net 3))
 (segment (start 83.82 93.98) (end 83.775455 93.935455) (width 0.2) (layer "F.Cu") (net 3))
 (segment (start 79.965372 91.48741) (end 84.799852 91.48741) (width 0.2) (layer "F.Cu") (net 1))
 (segment (start 79.873417 91.395455) (end 79.965372 91.48741) (width 0.2) (layer "F.Cu") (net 1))
 (segment (start 84.799852 91.48741) (end 85.812425 92.499983) (width 0.2) (layer "F.Cu") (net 1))
 (segment (start 73.66 124.46) (end 76.2 124.46) (width 0.2) (layer "F.Cu") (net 22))
 (segment (start 58.42 75.75396) (end 58.42 81.28) (width 0.2) (layer "F.Cu") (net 22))
 (segment (start 64.633417 71.028045) (end 63.145915 71.028045) (width 0.2) (layer "F.Cu") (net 22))
 (segment (start 58.42 81.28) (end 55.88 83.82) (width 0.2) (layer "F.Cu") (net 22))
 (segment (start 63.145915 71.028045) (end 58.42 75.75396) (width 0.2) (layer "F.Cu") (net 22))
 (segment (start 55.88 106.68) (end 73.66 124.46) (width 0.2) (layer "F.Cu") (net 22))
 (segment (start 55.88 83.82) (end 55.88 106.68) (width 0.2) (layer "F.Cu") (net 22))
 (segment (start 64.541462 78.74) (end 64.633417 78.648045) (width 0.2) (layer "F.Cu") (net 29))
 (segment (start 61.617641 83.728045) (end 58.82 86.525686) (width 0.2) (layer "F.Cu") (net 27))
 (segment (start 61.563737 83.674141) (end 61.617641 83.728045) (width 0.2) (layer "F.Cu") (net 27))
 (segment (start 64.633417 76.108045) (end 61.563737 79.177725) (width 0.2) (layer "F.Cu") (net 27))
 (segment (start 58.82 86.525686) (end 58.82 102) (width 0.2) (layer "F.Cu") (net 27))
 (segment (start 58.82 102) (end 83.82 127) (width 0.2) (layer "F.Cu") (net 27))
 (segment (start 61.563737 79.177725) (end 61.563737 83.674141) (width 0.2) (layer "F.Cu") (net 27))
 (segment (start 98.609054 48.14526) (end 98.609054 64.130823) (width 0.2) (layer "F.Cu") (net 18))
 (segment (start 98.389246 47.589246) (end 98.777157 47.977157) (width 0.2) (layer "F.Cu") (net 18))
 (segment (start 69.29876 50.08124) (end 69.29876 47.589246) (width 0.2) (layer "F.Cu") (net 18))
 (segment (start 69.29876 47.589246) (end 98.389246 47.589246) (width 0.2) (layer "F.Cu") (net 18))
 (segment (start 66.131955 53.248045) (end 69.29876 50.08124) (width 0.2) (layer "F.Cu") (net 18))
 (segment (start 64.633417 53.248045) (end 66.131955 53.248045) (width 0.2) (layer "F.Cu") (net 18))
 (segment (start 98.609054 64.130823) (end 99.009054 64.530823) (width 0.2) (layer "F.Cu") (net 18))
 (segment (start 98.777157 47.977157) (end 98.609054 48.14526) (width 0.2) (layer "F.Cu") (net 18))
 (segment (start 72.197679 54.802321) (end 72.197679 51.696636) (width 0.2) (layer "F.Cu") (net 19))
 (segment (start 72.197679 51.696636) (end 74.145671 49.748644) (width 0.2) (layer "F.Cu") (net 19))
 (segment (start 104.14 104.14) (end 104.14 106.68) (width 0.2) (layer "F.Cu") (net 19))
 (segment (start 94.972454 51.226769) (end 94.972454 94.972454) (width 0.2) (layer "F.Cu") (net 19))
 (segment (start 93.494329 49.748644) (end 94.972454 51.226769) (width 0.2) (layer "F.Cu") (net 19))
 (segment (start 66.131955 60.868045) (end 72.197679 54.802321) (width 0.2) (layer "F.Cu") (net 19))
 (segment (start 74.145671 49.748644) (end 93.494329 49.748644) (width 0.2) (layer "F.Cu") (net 19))
 (segment (start 104.14 106.68) (end 104.18 106.72) (width 0.2) (layer "F.Cu") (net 19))
 (segment (start 64.633417 60.868045) (end 66.131955 60.868045) (width 0.2) (layer "F.Cu") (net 19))
 (segment (start 94.972454 94.972454) (end 104.14 104.14) (width 0.2) (layer "F.Cu") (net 19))
 (segment (start 104.18 106.72) (end 104.18 111.539427) (width 0.2) (layer "F.Cu") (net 19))
 (segment (start 64.541462 73.66) (end 63.5 73.66) (width 0.2) (layer "F.Cu") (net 21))
 (segment (start 64.633417 73.568045) (end 64.541462 73.66) (width 0.2) (layer "F.Cu") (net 21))
 (segment (start 64.540279 73.661183) (end 64.633417 73.568045) (width 0.2) (layer "F.Cu") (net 21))
 (segment (start 59.956323 82.714558) (end 57.326691 85.34419) (width 0.2) (layer "F.Cu") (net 21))
 (segment (start 57.326691 85.34419) (end 57.446346 85.463845) (width 0.2) (layer "F.Cu") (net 21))
 (segment (start 57.446346 105.706346) (end 73.66 121.92) (width 0.2) (layer "F.Cu") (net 21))
 (segment (start 60.96 76.270955) (end 59.956323 77.274632) (width 0.2) (layer "F.Cu") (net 21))
 (segment (start 73.66 121.92) (end 76.2 121.92) (width 0.2) (layer "F.Cu") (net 21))
 (segment (start 63.5 73.66) (end 60.96 76.2) (width 0.2) (layer "F.Cu") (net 21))
 (segment (start 60.96 76.2) (end 60.96 76.270955) (width 0.2) (layer "F.Cu") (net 21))
 (segment (start 59.956323 77.274632) (end 59.956323 82.714558) (width 0.2) (layer "F.Cu") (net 21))
 (segment (start 57.446346 85.463845) (end 57.446346 105.706346) (width 0.2) (layer "F.Cu") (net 21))
 (segment (start 88.9 121.92) (end 88.9 118.814314) (width 0.2) (layer "F.Cu") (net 11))
 (segment (start 91.44 124.46) (end 88.9 121.92) (width 0.2) (layer "F.Cu") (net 11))
 (segment (start 79.828872 66.04) (end 79.873417 65.995455) (width 0.2) (layer "F.Cu") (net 11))
 (segment (start 88.9 118.814314) (end 71.12 101.034314) (width 0.2) (layer "F.Cu") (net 11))
 (segment (start 71.12 101.034314) (end 71.12 73.66) (width 0.2) (layer "F.Cu") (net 11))
 (segment (start 71.12 73.66) (end 78.74 66.04) (width 0.2) (layer "F.Cu") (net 11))
 (segment (start 78.74 66.04) (end 79.828872 66.04) (width 0.2) (layer "F.Cu") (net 11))
 (segment (start 79.917962 53.34) (end 79.873417 53.295455) (width 0.2) (layer "F.Cu") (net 16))
 (segment (start 83.82 53.34) (end 79.917962 53.34) (width 0.2) (layer "F.Cu") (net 16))
 (segment (start 84.277054 64.530823) (end 84.277054 53.797054) (width 0.2) (layer "F.Cu") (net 16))
 (segment (start 84.277054 53.797054) (end 83.82 53.34) (width 0.2) (layer "F.Cu") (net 16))
 (segment (start 96.12 121.52) (end 93.248628 118.648628) (width 0.2) (layer "F.Cu") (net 10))
 (segment (start 96.12 124.625685) (end 96.12 121.52) (width 0.2) (layer "F.Cu") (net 10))
 (segment (start 78.74 68.58) (end 79.828872 68.58) (width 0.2) (layer "F.Cu") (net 10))
 (segment (start 79.828872 68.58) (end 79.873417 68.535455) (width 0.2) (layer "F.Cu") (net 10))
 (segment (start 93.248628 118.648628) (end 90.991471 118.648628) (width 0.2) (layer "F.Cu") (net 10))
 (segment (start 96.52 129.54) (end 96.52 125.025685) (width 0.2) (layer "F.Cu") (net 10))
 (segment (start 73.66 101.317157) (end 73.66 73.66) (width 0.2) (layer "F.Cu") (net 10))
 (segment (start 99.06 129.54) (end 96.52 129.54) (width 0.2) (layer "F.Cu") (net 10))
 (segment (start 90.991471 118.648628) (end 73.66 101.317157) (width 0.2) (layer "F.Cu") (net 10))
 (segment (start 96.52 125.025685) (end 96.12 124.625685) (width 0.2) (layer "F.Cu") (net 10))
 (segment (start 73.66 73.66) (end 78.74 68.58) (width 0.2) (layer "F.Cu") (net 10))
 (segment (start 79.873417 73.615455) (end 83.201686 73.615455) (width 0.2) (layer "F.Cu") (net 8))
 (segment (start 83.201686 73.615455) (end 84.277054 74.690823) (width 0.2) (layer "F.Cu") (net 8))
 (segment (start 84.277054 74.690823) (end 84.277054 74.117054) (width 0.2) (layer "F.Cu") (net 8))
 (segment (start 76.2 99.06) (end 76.2 73.70741) (width 0.2) (layer "F.Cu") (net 9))
 (segment (start 90.17 117.261471) (end 78.74 105.831471) (width 0.2) (layer "F.Cu") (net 9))
 (segment (start 78.74 101.6) (end 76.2 99.06) (width 0.2) (layer "F.Cu") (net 9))
 (segment (start 96.52 124.46) (end 96.52 121.354315) (width 0.2) (layer "F.Cu") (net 9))
 (segment (start 76.2 73.70741) (end 78.74 71.16741) (width 0.2) (layer "F.Cu") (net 9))
 (segment (start 92.427156 117.261471) (end 90.17 117.261471) (width 0.2) (layer "F.Cu") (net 9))
 (segment (start 78.69259 71.16741) (end 78.74 71.16741) (width 0.2) (layer "F.Cu") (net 9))
 (segment (start 78.74 71.16741) (end 79.781462 71.16741) (width 0.2) (layer "F.Cu") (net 9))
 (segment (start 99.06 124.46) (end 96.52 124.46) (width 0.2) (layer "F.Cu") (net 9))
 (segment (start 78.74 105.831471) (end 78.74 101.6) (width 0.2) (layer "F.Cu") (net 9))
 (segment (start 79.781462 71.16741) (end 79.873417 71.075455) (width 0.2) (layer "F.Cu") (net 9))
 (segment (start 96.52 121.354315) (end 92.427156 117.261471) (width 0.2) (layer "F.Cu") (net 9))
 (segment (start 64.541462 86.36) (end 64.633417 86.268045) (width 0.2) (layer "F.Cu") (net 30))
 (segment (start 60.96 101.6) (end 60.96 88.9) (width 0.2) (layer "F.Cu") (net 26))
 (segment (start 61.051955 88.808045) (end 64.633417 88.808045) (width 0.2) (layer "F.Cu") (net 26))
 (segment (start 83.82 124.46) (end 60.96 101.6) (width 0.2) (layer "F.Cu") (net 26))
 (segment (start 60.96 88.9) (end 61.051955 88.808045) (width 0.2) (layer "F.Cu") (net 26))
 (segment (start 64.541462 88.9) (end 64.633417 88.808045) (width 0.2) (layer "F.Cu") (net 26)))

